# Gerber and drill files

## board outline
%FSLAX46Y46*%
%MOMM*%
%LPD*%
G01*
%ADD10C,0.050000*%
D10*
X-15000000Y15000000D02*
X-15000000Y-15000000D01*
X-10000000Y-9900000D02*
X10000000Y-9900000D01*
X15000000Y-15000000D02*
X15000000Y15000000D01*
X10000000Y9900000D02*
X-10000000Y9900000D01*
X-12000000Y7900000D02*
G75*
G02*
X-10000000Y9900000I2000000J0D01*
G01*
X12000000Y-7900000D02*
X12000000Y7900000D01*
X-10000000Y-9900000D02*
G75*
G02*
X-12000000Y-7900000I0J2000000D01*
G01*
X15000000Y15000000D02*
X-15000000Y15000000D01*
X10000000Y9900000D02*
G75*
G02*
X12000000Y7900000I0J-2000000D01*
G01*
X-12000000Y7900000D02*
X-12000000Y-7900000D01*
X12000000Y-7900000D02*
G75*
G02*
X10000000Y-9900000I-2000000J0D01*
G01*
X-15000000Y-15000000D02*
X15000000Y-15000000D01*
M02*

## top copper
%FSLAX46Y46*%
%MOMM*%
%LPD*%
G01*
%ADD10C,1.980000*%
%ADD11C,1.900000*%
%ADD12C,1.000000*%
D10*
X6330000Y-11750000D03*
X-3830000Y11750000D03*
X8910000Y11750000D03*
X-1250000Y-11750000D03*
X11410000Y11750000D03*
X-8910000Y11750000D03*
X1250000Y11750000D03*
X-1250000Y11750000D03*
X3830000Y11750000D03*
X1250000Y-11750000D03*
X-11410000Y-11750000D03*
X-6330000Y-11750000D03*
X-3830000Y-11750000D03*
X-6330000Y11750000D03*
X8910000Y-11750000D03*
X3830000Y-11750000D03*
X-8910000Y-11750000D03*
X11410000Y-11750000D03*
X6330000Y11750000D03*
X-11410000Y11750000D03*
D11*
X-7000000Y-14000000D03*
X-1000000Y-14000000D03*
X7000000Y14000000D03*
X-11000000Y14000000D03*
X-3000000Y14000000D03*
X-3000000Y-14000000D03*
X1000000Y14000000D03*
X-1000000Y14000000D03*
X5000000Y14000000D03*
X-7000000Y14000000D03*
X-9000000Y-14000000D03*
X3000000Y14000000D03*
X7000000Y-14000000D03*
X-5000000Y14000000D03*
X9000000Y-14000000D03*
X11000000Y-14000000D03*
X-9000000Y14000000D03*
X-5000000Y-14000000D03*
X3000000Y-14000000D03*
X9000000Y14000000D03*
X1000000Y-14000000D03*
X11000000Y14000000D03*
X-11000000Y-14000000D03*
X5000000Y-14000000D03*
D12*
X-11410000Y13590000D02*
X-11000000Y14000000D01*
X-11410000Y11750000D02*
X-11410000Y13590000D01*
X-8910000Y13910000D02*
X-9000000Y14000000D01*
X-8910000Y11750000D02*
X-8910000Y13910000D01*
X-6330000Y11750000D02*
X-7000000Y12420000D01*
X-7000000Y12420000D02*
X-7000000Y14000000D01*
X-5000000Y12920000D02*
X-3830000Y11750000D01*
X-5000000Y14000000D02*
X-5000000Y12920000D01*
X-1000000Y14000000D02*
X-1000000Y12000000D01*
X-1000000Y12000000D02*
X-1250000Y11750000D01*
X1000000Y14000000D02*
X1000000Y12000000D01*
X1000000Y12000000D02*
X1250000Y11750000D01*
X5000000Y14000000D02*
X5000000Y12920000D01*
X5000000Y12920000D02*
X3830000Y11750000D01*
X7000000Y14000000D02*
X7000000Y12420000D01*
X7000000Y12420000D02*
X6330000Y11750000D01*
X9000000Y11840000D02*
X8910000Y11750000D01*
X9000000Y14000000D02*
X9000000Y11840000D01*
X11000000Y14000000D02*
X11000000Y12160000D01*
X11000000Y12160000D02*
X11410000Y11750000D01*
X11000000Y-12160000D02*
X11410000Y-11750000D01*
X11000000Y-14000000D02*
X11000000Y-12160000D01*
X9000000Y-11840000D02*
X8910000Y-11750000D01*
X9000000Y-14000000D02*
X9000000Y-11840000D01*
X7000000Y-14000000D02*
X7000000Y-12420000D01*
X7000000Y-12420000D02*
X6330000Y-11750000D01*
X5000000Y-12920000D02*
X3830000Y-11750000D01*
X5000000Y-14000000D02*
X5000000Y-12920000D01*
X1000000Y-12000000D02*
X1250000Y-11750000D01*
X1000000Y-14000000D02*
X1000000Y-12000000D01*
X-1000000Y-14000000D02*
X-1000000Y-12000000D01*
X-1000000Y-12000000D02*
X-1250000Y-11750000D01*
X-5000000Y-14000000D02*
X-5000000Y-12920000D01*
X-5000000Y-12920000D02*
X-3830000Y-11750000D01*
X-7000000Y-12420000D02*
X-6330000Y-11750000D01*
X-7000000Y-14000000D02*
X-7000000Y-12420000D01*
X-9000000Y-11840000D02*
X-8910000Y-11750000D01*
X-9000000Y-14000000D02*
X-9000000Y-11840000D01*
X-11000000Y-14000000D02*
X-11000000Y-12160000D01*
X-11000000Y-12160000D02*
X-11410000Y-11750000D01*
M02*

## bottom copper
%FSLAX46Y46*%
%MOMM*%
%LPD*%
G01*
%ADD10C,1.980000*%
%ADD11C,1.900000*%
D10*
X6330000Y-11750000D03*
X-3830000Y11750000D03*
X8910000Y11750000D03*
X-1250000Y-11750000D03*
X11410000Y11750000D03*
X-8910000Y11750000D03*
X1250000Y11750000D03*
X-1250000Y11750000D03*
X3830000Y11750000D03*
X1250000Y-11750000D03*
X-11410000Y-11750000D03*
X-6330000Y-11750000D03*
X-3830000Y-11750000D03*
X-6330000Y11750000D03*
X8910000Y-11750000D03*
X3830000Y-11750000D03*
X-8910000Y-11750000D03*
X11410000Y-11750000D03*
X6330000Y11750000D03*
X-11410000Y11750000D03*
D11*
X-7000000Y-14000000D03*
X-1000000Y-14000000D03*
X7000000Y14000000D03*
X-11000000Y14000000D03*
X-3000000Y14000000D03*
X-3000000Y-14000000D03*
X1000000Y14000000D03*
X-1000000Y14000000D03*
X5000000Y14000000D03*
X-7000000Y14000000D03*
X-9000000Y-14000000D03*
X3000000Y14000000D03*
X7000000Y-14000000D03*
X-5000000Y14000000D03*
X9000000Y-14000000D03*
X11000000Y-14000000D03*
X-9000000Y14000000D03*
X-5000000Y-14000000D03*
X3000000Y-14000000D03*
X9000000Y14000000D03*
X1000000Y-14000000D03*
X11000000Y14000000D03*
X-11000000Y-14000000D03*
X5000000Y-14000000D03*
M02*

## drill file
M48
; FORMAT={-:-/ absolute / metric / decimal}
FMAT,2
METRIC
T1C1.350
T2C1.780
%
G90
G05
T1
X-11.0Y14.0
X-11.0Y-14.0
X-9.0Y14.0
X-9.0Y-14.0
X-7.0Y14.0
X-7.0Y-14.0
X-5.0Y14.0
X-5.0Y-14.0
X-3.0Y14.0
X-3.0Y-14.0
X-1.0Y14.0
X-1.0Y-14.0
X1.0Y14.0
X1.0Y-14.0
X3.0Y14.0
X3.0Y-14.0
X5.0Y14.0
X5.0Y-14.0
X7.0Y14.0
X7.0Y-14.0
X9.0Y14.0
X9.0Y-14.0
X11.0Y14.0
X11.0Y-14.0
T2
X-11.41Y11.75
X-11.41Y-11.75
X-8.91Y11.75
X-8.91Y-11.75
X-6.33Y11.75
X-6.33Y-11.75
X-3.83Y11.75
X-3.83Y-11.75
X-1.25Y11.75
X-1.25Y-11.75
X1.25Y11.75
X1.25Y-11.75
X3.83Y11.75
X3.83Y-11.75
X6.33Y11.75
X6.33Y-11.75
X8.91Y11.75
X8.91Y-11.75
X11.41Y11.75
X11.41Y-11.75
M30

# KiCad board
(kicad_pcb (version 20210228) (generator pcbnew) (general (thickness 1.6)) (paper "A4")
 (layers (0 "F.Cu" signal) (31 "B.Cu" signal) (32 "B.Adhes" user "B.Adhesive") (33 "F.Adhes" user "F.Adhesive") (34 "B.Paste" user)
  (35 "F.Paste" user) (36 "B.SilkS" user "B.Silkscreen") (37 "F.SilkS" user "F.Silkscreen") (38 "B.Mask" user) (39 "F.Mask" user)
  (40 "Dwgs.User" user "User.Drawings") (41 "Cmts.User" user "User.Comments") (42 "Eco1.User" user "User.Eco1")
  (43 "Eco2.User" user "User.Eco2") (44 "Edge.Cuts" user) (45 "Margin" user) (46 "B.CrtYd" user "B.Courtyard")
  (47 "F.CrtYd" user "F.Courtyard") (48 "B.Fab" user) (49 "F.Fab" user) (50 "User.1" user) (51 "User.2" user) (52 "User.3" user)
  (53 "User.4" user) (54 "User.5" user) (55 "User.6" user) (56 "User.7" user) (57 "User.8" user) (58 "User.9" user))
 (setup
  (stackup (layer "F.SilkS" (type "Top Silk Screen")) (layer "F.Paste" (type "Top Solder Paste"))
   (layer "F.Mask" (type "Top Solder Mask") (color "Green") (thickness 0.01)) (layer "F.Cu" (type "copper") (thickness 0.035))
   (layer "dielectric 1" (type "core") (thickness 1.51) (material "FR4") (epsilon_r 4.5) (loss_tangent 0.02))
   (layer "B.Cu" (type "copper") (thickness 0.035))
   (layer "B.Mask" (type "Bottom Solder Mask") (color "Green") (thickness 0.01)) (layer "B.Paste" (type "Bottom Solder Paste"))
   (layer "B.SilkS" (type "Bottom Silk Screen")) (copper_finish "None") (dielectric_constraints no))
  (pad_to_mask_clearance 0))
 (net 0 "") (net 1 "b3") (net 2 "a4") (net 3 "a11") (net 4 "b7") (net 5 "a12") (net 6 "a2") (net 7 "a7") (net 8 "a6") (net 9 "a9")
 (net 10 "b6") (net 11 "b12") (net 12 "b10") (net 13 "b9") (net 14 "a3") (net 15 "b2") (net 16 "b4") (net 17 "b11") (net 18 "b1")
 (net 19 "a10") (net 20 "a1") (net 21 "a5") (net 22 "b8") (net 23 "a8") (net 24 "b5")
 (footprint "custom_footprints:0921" (layer "F.Cu") (at 6.33 11.75)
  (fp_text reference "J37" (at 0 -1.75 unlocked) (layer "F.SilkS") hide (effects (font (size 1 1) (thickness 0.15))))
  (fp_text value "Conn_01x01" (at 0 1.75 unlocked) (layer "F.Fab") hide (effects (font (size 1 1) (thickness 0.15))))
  (pad "1" thru_hole circle (at 0 0) (size 1.98 1.98) (drill 1.78) (layers *.Cu *.Mask) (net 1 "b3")))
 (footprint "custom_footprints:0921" (layer "F.Cu") (at -3.83 -11.75)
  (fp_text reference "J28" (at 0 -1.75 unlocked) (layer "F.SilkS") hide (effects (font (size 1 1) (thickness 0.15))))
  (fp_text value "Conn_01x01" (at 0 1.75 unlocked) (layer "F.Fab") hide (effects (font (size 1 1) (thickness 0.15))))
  (pad "1" thru_hole circle (at 0 0) (size 1.98 1.98) (drill 1.78) (layers *.Cu *.Mask) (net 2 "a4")))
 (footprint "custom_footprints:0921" (layer "F.Cu") (at 8.91 -11.75)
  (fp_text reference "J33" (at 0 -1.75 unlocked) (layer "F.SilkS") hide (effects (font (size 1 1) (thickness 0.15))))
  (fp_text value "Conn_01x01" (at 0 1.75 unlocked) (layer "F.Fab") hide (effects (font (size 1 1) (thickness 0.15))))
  (pad "1" thru_hole circle (at 0 0) (size 1.98 1.98) (drill 1.78) (layers *.Cu *.Mask) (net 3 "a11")))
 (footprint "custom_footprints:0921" (layer "F.Cu") (at -1.25 11.75)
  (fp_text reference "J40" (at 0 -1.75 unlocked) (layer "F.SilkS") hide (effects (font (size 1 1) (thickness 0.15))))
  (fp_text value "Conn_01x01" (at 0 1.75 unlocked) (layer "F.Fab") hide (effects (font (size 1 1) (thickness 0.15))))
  (pad "1" thru_hole circle (at 0 0) (size 1.98 1.98) (drill 1.78) (layers *.Cu *.Mask) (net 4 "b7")))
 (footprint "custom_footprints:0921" (layer "F.Cu") (at 11.41 -11.75)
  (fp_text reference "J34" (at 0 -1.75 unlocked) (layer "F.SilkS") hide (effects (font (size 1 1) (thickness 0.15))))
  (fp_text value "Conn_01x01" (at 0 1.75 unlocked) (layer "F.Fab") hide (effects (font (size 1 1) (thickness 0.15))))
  (pad "1" thru_hole circle (at 0 0) (size 1.98 1.98) (drill 1.78) (layers *.Cu *.Mask) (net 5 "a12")))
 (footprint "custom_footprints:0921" (layer "F.Cu") (at -8.91 -11.75)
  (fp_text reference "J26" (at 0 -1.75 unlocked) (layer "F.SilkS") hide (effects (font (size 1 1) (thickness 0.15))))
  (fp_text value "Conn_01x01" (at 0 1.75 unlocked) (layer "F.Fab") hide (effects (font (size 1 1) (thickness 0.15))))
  (pad "1" thru_hole circle (at 0 0) (size 1.98 1.98) (drill 1.78) (layers *.Cu *.Mask) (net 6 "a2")))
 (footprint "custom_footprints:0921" (layer "F.Cu") (at 1.25 -11.75)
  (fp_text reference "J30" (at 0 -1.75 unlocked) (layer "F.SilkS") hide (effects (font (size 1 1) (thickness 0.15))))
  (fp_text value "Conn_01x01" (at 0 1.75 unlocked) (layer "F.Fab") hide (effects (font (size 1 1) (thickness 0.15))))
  (pad "1" thru_hole circle (at 0 0) (size 1.98 1.98) (drill 1.78) (layers *.Cu *.Mask) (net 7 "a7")))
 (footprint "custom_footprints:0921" (layer "F.Cu") (at -1.25 -11.75)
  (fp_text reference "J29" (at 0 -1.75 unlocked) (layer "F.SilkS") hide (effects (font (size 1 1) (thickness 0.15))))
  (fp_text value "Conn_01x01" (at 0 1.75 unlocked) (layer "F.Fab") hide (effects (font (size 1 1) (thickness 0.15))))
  (pad "1" thru_hole circle (at 0 0) (size 1.98 1.98) (drill 1.78) (layers *.Cu *.Mask) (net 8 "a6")))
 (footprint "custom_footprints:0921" (layer "F.Cu") (at 3.83 -11.75)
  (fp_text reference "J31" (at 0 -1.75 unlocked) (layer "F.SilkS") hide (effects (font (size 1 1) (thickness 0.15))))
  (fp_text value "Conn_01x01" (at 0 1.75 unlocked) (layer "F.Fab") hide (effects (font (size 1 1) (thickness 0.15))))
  (pad "1" thru_hole circle (at 0 0) (size 1.98 1.98) (drill 1.78) (layers *.Cu *.Mask) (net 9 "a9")))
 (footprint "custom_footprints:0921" (layer "F.Cu") (at 1.25 11.75)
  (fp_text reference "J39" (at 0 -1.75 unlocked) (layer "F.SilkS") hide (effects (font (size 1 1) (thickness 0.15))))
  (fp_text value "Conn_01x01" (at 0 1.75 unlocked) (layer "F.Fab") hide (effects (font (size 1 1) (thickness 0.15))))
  (pad "1" thru_hole circle (at 0 0) (size 1.98 1.98) (drill 1.78) (layers *.Cu *.Mask) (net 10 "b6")))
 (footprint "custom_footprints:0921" (layer "F.Cu") (at -11.41 11.75)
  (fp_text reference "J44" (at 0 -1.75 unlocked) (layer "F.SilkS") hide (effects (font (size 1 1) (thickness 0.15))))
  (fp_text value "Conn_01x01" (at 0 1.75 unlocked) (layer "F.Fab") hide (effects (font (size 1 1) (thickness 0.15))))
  (pad "1" thru_hole circle (at 0 0) (size 1.98 1.98) (drill 1.78) (layers *.Cu *.Mask) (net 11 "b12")))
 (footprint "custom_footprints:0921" (layer "F.Cu") (at -6.33 11.75)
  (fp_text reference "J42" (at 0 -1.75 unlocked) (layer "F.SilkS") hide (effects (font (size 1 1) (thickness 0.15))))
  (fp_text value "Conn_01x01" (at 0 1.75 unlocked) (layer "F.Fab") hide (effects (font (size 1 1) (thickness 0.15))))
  (pad "1" thru_hole circle (at 0 0) (size 1.98 1.98) (drill 1.78) (layers *.Cu *.Mask) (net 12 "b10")))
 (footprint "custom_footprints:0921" (layer "F.Cu") (at -3.83 11.75)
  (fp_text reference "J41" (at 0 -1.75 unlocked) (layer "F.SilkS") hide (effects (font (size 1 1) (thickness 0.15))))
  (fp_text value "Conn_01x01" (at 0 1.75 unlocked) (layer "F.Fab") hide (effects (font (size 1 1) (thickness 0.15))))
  (pad "1" thru_hole circle (at 0 0) (size 1.98 1.98) (drill 1.78) (layers *.Cu *.Mask) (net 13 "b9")))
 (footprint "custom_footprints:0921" (layer "F.Cu") (at -6.33 -11.75)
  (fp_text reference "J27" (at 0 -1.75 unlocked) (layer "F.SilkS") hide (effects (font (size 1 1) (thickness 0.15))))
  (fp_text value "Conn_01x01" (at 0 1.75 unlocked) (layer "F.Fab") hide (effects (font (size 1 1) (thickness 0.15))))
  (pad "1" thru_hole circle (at 0 0) (size 1.98 1.98) (drill 1.78) (layers *.Cu *.Mask) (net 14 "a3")))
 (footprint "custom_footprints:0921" (layer "F.Cu") (at 8.91 11.75)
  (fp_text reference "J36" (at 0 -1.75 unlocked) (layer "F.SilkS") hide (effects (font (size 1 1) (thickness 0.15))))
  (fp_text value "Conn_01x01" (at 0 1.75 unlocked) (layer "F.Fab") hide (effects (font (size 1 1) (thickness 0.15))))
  (pad "1" thru_hole circle (at 0 0) (size 1.98 1.98) (drill 1.78) (layers *.Cu *.Mask) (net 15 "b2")))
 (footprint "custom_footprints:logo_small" (layer "F.Cu") (at -14 -4 90)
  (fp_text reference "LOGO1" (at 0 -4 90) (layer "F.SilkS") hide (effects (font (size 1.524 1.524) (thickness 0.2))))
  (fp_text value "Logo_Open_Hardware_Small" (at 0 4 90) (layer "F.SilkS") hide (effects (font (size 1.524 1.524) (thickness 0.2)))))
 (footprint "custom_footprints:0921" (layer "F.Cu") (at 3.83 11.75)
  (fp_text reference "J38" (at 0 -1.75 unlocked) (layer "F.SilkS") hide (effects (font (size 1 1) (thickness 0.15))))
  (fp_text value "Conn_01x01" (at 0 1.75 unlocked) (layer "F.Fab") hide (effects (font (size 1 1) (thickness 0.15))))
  (pad "1" thru_hole circle (at 0 0) (size 1.98 1.98) (drill 1.78) (layers *.Cu *.Mask) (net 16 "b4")))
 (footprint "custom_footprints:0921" (layer "F.Cu") (at -8.91 11.75)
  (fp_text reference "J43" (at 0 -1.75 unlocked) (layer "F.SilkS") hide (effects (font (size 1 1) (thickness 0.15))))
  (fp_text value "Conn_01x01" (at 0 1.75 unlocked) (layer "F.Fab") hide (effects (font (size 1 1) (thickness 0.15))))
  (pad "1" thru_hole circle (at 0 0) (size 1.98 1.98) (drill 1.78) (layers *.Cu *.Mask) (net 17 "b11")))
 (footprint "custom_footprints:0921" (layer "F.Cu") (at 11.41 11.75)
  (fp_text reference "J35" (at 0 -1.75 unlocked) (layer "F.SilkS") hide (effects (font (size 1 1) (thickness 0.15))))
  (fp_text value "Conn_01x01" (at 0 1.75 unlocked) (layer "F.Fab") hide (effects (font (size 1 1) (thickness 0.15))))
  (pad "1" thru_hole circle (at 0 0) (size 1.98 1.98) (drill 1.78) (layers *.Cu *.Mask) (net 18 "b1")))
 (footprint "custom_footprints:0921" (layer "F.Cu") (at 6.33 -11.75)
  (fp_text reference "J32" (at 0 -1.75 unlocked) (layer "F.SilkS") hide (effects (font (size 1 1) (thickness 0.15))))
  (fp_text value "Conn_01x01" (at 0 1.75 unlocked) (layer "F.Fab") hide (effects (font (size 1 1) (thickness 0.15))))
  (pad "1" thru_hole circle (at 0 0) (size 1.98 1.98) (drill 1.78) (layers *.Cu *.Mask) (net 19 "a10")))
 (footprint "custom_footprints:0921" (layer "F.Cu") (at -11.41 -11.75)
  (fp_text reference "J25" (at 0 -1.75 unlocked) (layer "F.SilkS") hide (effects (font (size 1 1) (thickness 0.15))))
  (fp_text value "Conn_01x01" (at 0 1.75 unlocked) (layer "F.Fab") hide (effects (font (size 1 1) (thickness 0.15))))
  (pad "1" thru_hole circle (at 0 0) (size 1.98 1.98) (drill 1.78) (layers *.Cu *.Mask) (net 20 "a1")))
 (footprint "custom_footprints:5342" (layer "B.Cu") (at -7 14)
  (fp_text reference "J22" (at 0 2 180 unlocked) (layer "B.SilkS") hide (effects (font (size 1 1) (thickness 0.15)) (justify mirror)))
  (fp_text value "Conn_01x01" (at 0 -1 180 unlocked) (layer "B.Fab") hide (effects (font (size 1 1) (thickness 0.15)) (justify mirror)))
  (pad "1" thru_hole circle (at 0 0) (size 1.9 1.9) (drill 1.35) (layers *.Cu *.Mask) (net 12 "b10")))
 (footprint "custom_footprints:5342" (layer "B.Cu") (at -1 14)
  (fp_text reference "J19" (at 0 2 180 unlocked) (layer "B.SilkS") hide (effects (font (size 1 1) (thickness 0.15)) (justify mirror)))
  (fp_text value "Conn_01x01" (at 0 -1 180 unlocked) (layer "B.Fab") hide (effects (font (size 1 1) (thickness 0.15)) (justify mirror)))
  (pad "1" thru_hole circle (at 0 0) (size 1.9 1.9) (drill 1.35) (layers *.Cu *.Mask) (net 4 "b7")))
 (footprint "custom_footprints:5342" (layer "B.Cu") (at 7 -14)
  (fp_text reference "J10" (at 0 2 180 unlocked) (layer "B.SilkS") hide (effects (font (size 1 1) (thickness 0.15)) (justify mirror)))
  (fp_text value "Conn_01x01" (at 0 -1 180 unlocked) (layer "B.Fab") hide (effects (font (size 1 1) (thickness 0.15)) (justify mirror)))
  (pad "1" thru_hole circle (at 0 0) (size 1.9 1.9) (drill 1.35) (layers *.Cu *.Mask) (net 19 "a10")))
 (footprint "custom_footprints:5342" (layer "B.Cu") (at -11 -14)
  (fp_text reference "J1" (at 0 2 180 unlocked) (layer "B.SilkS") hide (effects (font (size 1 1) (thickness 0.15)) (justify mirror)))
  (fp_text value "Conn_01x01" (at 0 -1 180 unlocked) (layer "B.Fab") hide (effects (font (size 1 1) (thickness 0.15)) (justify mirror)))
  (pad "1" thru_hole circle (at 0 0) (size 1.9 1.9) (drill 1.35) (layers *.Cu *.Mask) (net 20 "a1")))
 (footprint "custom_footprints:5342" (layer "B.Cu") (at -3 -14)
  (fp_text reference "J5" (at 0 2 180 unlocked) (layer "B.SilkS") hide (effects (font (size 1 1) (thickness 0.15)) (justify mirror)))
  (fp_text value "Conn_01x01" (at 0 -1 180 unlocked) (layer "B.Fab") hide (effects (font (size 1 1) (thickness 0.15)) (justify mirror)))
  (pad "1" thru_hole circle (at 0 0) (size 1.9 1.9) (drill 1.35) (layers *.Cu *.Mask) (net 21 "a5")))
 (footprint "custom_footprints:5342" (layer "B.Cu") (at -3 14)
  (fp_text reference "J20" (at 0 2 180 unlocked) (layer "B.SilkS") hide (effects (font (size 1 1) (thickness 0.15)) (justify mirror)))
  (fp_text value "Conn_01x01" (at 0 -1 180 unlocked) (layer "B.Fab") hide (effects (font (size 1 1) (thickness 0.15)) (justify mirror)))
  (pad "1" thru_hole circle (at 0 0) (size 1.9 1.9) (drill 1.35) (layers *.Cu *.Mask) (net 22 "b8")))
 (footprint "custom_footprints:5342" (layer "B.Cu") (at 1 -14)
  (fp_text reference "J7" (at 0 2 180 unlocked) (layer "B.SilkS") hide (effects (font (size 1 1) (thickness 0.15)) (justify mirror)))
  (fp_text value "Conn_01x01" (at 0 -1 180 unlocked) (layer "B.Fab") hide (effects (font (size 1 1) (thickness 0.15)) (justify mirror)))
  (pad "1" thru_hole circle (at 0 0) (size 1.9 1.9) (drill 1.35) (layers *.Cu *.Mask) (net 7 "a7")))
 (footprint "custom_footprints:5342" (layer "B.Cu") (at -1 -14)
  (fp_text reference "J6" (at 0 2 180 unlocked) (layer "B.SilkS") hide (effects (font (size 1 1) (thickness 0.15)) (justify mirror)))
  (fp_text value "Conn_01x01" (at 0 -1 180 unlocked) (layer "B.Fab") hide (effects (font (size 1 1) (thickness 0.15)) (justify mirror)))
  (pad "1" thru_hole circle (at 0 0) (size 1.9 1.9) (drill 1.35) (layers *.Cu *.Mask) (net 8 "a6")))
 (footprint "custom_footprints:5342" (layer "B.Cu") (at 5 -14)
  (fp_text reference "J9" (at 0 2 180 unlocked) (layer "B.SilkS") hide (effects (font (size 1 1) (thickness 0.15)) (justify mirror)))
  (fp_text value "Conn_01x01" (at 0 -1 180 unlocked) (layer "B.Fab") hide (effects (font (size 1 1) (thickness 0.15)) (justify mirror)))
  (pad "1" thru_hole circle (at 0 0) (size 1.9 1.9) (drill 1.35) (layers *.Cu *.Mask) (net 9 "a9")))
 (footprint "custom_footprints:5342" (layer "B.Cu") (at -7 -14)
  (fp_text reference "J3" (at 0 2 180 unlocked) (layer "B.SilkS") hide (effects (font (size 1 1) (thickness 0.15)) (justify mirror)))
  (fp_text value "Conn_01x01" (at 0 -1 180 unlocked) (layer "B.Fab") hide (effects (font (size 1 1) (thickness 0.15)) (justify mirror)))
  (pad "1" thru_hole circle (at 0 0) (size 1.9 1.9) (drill 1.35) (layers *.Cu *.Mask) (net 14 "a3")))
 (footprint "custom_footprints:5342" (layer "B.Cu") (at -9 14)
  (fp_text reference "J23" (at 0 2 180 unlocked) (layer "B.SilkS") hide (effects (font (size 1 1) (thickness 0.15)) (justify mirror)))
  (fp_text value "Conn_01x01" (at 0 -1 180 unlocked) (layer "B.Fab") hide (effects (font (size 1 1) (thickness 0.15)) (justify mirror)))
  (pad "1" thru_hole circle (at 0 0) (size 1.9 1.9) (drill 1.35) (layers *.Cu *.Mask) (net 17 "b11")))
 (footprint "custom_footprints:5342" (layer "B.Cu") (at 3 -14)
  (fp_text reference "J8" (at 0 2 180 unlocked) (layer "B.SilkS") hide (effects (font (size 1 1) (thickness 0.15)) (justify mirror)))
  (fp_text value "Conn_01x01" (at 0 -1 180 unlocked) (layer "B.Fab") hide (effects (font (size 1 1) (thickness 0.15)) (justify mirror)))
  (pad "1" thru_hole circle (at 0 0) (size 1.9 1.9) (drill 1.35) (layers *.Cu *.Mask) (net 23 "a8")))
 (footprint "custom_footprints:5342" (layer "B.Cu") (at 7 14)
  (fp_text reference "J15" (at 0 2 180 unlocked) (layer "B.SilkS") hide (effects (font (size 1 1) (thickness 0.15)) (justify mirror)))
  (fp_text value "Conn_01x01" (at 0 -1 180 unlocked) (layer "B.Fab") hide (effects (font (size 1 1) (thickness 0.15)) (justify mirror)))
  (pad "1" thru_hole circle (at 0 0) (size 1.9 1.9) (drill 1.35) (layers *.Cu *.Mask) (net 1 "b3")))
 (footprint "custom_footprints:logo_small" (layer "B.Cu") (at -14 -4 -90)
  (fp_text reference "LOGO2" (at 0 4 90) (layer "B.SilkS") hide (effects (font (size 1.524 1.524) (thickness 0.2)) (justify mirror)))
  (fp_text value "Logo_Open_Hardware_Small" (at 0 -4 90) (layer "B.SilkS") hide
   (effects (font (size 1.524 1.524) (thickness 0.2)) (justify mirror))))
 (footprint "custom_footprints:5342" (layer "B.Cu") (at -5 -14)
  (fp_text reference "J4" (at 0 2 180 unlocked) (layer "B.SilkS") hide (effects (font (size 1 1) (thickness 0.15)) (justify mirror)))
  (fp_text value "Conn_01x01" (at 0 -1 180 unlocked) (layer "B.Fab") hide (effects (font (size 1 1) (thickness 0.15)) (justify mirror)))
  (pad "1" thru_hole circle (at 0 0) (size 1.9 1.9) (drill 1.35) (layers *.Cu *.Mask) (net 2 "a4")))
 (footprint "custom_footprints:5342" (layer "B.Cu") (at 9 14)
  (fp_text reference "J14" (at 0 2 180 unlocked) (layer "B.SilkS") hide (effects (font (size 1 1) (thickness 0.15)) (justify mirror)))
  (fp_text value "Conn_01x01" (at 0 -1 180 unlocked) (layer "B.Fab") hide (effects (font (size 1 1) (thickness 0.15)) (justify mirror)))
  (pad "1" thru_hole circle (at 0 0) (size 1.9 1.9) (drill 1.35) (layers *.Cu *.Mask) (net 15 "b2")))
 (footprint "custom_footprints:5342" (layer "B.Cu") (at 11 14)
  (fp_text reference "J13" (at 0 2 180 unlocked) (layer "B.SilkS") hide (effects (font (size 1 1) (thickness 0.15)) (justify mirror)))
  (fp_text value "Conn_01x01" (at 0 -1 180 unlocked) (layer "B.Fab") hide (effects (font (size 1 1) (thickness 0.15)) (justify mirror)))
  (pad "1" thru_hole circle (at 0 0) (size 1.9 1.9) (drill 1.35) (layers *.Cu *.Mask) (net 18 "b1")))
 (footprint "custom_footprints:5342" (layer "B.Cu") (at -9 -14)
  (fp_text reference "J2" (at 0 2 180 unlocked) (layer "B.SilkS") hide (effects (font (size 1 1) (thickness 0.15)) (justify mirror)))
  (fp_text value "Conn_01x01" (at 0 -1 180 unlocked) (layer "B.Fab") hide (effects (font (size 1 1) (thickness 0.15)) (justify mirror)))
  (pad "1" thru_hole circle (at 0 0) (size 1.9 1.9) (drill 1.35) (layers *.Cu *.Mask) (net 6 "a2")))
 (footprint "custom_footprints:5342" (layer "B.Cu") (at -5 14)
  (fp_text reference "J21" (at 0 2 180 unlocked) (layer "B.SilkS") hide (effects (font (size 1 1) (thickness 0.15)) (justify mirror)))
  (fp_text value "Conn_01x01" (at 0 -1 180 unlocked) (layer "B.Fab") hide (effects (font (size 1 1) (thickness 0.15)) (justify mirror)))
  (pad "1" thru_hole circle (at 0 0) (size 1.9 1.9) (drill 1.35) (layers *.Cu *.Mask) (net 13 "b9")))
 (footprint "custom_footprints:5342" (layer "B.Cu") (at 3 14)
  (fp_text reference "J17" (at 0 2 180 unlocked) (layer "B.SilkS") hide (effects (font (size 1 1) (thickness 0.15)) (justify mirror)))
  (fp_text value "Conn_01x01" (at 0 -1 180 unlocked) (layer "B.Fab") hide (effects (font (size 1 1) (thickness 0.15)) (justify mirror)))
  (pad "1" thru_hole circle (at 0 0) (size 1.9 1.9) (drill 1.35) (layers *.Cu *.Mask) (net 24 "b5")))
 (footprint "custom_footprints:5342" (layer "B.Cu") (at 9 -14)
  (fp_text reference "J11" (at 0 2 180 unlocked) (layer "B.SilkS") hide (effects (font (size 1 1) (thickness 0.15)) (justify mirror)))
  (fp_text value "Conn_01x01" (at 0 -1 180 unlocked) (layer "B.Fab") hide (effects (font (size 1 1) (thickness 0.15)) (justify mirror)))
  (pad "1" thru_hole circle (at 0 0) (size 1.9 1.9) (drill 1.35) (layers *.Cu *.Mask) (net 3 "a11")))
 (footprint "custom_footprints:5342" (layer "B.Cu") (at 1 14)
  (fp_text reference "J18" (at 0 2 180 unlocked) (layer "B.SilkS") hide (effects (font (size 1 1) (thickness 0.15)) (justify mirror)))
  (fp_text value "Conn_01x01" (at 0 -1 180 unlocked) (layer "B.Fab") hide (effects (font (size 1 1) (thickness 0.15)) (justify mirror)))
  (pad "1" thru_hole circle (at 0 0) (size 1.9 1.9) (drill 1.35) (layers *.Cu *.Mask) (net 10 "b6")))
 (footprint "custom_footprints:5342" (layer "B.Cu") (at 11 -14)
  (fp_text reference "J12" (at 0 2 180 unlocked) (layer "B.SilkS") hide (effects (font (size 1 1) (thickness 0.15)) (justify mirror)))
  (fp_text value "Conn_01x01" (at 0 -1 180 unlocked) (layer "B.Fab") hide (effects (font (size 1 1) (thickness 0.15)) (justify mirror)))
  (pad "1" thru_hole circle (at 0 0) (size 1.9 1.9) (drill 1.35) (layers *.Cu *.Mask) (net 5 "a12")))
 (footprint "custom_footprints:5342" (layer "B.Cu") (at -11 14)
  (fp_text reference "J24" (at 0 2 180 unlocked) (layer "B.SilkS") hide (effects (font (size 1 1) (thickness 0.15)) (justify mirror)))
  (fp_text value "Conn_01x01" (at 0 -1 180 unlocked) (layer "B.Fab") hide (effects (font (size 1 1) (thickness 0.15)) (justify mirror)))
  (pad "1" thru_hole circle (at 0 0) (size 1.9 1.9) (drill 1.35) (layers *.Cu *.Mask) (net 11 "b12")))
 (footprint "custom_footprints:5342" (layer "B.Cu") (at 5 14)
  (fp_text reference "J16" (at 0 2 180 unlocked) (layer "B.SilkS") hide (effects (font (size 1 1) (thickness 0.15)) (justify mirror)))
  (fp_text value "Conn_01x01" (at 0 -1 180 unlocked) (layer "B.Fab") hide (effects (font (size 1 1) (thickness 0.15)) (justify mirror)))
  (pad "1" thru_hole circle (at 0 0) (size 1.9 1.9) (drill 1.35) (layers *.Cu *.Mask) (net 16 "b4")))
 (gr_line (start -15 -15) (end -15 15) (layer "Edge.Cuts") (width 0.05))
 (gr_line (start -10 9.9) (end 10 9.9) (layer "Edge.Cuts") (width 0.05))
 (gr_line (start 15 15) (end 15 -15) (layer "Edge.Cuts") (width 0.05))
 (gr_line (start 10 -9.9) (end -10 -9.9) (layer "Edge.Cuts") (width 0.05))
 (gr_arc (start -10 -7.9) (end -10 -9.9) (angle -90) (layer "Edge.Cuts") (width 0.05))
 (gr_line (start 12 7.9) (end 12 -7.9) (layer "Edge.Cuts") (width 0.05))
 (gr_arc (start -10 7.9) (end -12 7.9) (angle -90) (layer "Edge.Cuts") (width 0.05))
 (gr_line (start 15 -15) (end -15 -15) (layer "Edge.Cuts") (width 0.05))
 (gr_arc (start 10 -7.9) (end 12 -7.9) (angle -90) (layer "Edge.Cuts") (width 0.05))
 (gr_line (start -12 -7.9) (end -12 7.9) (layer "Edge.Cuts") (width 0.05))
 (gr_arc (start 10 7.9) (end 10 9.9) (angle -90) (layer "Edge.Cuts") (width 0.05))
 (gr_line (start -15 15) (end 15 15) (layer "Edge.Cuts") (width 0.05))
 (segment (start -11.41 -13.59) (end -11 -14) (width 1) (layer "F.Cu") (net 20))
 (segment (start -11.41 -11.75) (end -11.41 -13.59) (width 1) (layer "F.Cu") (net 20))
 (segment (start -8.91 -13.91) (end -9 -14) (width 1) (layer "F.Cu") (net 6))
 (segment (start -8.91 -11.75) (end -8.91 -13.91) (width 1) (layer "F.Cu") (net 6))
 (segment (start -6.33 -11.75) (end -7 -12.42) (width 1) (layer "F.Cu") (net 14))
 (segment (start -7 -12.42) (end -7 -14) (width 1) (layer "F.Cu") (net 14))
 (segment (start -5 -12.92) (end -3.83 -11.75) (width 1) (layer "F.Cu") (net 2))
 (segment (start -5 -14) (end -5 -12.92) (width 1) (layer "F.Cu") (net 2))
 (segment (start -1 -14) (end -1 -12) (width 1) (layer "F.Cu") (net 8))
 (segment (start -1 -12) (end -1.25 -11.75) (width 1) (layer "F.Cu") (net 8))
 (segment (start 1 -14) (end 1 -12) (width 1) (layer "F.Cu") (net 7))
 (segment (start 1 -12) (end 1.25 -11.75) (width 1) (layer "F.Cu") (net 7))
 (segment (start 5 -14) (end 5 -12.92) (width 1) (layer "F.Cu") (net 9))
 (segment (start 5 -12.92) (end 3.83 -11.75) (width 1) (layer "F.Cu") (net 9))
 (segment (start 7 -14) (end 7 -12.42) (width 1) (layer "F.Cu") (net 19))
 (segment (start 7 -12.42) (end 6.33 -11.75) (width 1) (layer "F.Cu") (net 19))
 (segment (start 9 -11.84) (end 8.91 -11.75) (width 1) (layer "F.Cu") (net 3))
 (segment (start 9 -14) (end 9 -11.84) (width 1) (layer "F.Cu") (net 3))
 (segment (start 11 -14) (end 11 -12.16) (width 1) (layer "F.Cu") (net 5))
 (segment (start 11 -12.16) (end 11.41 -11.75) (width 1) (layer "F.Cu") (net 5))
 (segment (start 11 12.16) (end 11.41 11.75) (width 1) (layer "F.Cu") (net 18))
 (segment (start 11 14) (end 11 12.16) (width 1) (layer "F.Cu") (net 18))
 (segment (start 9 11.84) (end 8.91 11.75) (width 1) (layer "F.Cu") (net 15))
 (segment (start 9 14) (end 9 11.84) (width 1) (layer "F.Cu") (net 15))
 (segment (start 7 14) (end 7 12.42) (width 1) (layer "F.Cu") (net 1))
 (segment (start 7 12.42) (end 6.33 11.75) (width 1) (layer "F.Cu") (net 1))
 (segment (start 5 12.92) (end 3.83 11.75) (width 1) (layer "F.Cu") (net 16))
 (segment (start 5 14) (end 5 12.92) (width 1) (layer "F.Cu") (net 16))
 (segment (start 1 12) (end 1.25 11.75) (width 1) (layer "F.Cu") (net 10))
 (segment (start 1 14) (end 1 12) (width 1) (layer "F.Cu") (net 10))
 (segment (start -1 14) (end -1 12) (width 1) (layer "F.Cu") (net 4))
 (segment (start -1 12) (end -1.25 11.75) (width 1) (layer "F.Cu") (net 4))
 (segment (start -5 14) (end -5 12.92) (width 1) (layer "F.Cu") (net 13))
 (segment (start -5 12.92) (end -3.83 11.75) (width 1) (layer "F.Cu") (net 13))
 (segment (start -7 12.42) (end -6.33 11.75) (width 1) (layer "F.Cu") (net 12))
 (segment (start -7 14) (end -7 12.42) (width 1) (layer "F.Cu") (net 12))
 (segment (start -9 11.84) (end -8.91 11.75) (width 1) (layer "F.Cu") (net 17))
 (segment (start -9 14) (end -9 11.84) (width 1) (layer "F.Cu") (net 17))
 (segment (start -11 14) (end -11 12.16) (width 1) (layer "F.Cu") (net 11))
 (segment (start -11 12.16) (end -11.41 11.75) (width 1) (layer "F.Cu") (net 11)))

